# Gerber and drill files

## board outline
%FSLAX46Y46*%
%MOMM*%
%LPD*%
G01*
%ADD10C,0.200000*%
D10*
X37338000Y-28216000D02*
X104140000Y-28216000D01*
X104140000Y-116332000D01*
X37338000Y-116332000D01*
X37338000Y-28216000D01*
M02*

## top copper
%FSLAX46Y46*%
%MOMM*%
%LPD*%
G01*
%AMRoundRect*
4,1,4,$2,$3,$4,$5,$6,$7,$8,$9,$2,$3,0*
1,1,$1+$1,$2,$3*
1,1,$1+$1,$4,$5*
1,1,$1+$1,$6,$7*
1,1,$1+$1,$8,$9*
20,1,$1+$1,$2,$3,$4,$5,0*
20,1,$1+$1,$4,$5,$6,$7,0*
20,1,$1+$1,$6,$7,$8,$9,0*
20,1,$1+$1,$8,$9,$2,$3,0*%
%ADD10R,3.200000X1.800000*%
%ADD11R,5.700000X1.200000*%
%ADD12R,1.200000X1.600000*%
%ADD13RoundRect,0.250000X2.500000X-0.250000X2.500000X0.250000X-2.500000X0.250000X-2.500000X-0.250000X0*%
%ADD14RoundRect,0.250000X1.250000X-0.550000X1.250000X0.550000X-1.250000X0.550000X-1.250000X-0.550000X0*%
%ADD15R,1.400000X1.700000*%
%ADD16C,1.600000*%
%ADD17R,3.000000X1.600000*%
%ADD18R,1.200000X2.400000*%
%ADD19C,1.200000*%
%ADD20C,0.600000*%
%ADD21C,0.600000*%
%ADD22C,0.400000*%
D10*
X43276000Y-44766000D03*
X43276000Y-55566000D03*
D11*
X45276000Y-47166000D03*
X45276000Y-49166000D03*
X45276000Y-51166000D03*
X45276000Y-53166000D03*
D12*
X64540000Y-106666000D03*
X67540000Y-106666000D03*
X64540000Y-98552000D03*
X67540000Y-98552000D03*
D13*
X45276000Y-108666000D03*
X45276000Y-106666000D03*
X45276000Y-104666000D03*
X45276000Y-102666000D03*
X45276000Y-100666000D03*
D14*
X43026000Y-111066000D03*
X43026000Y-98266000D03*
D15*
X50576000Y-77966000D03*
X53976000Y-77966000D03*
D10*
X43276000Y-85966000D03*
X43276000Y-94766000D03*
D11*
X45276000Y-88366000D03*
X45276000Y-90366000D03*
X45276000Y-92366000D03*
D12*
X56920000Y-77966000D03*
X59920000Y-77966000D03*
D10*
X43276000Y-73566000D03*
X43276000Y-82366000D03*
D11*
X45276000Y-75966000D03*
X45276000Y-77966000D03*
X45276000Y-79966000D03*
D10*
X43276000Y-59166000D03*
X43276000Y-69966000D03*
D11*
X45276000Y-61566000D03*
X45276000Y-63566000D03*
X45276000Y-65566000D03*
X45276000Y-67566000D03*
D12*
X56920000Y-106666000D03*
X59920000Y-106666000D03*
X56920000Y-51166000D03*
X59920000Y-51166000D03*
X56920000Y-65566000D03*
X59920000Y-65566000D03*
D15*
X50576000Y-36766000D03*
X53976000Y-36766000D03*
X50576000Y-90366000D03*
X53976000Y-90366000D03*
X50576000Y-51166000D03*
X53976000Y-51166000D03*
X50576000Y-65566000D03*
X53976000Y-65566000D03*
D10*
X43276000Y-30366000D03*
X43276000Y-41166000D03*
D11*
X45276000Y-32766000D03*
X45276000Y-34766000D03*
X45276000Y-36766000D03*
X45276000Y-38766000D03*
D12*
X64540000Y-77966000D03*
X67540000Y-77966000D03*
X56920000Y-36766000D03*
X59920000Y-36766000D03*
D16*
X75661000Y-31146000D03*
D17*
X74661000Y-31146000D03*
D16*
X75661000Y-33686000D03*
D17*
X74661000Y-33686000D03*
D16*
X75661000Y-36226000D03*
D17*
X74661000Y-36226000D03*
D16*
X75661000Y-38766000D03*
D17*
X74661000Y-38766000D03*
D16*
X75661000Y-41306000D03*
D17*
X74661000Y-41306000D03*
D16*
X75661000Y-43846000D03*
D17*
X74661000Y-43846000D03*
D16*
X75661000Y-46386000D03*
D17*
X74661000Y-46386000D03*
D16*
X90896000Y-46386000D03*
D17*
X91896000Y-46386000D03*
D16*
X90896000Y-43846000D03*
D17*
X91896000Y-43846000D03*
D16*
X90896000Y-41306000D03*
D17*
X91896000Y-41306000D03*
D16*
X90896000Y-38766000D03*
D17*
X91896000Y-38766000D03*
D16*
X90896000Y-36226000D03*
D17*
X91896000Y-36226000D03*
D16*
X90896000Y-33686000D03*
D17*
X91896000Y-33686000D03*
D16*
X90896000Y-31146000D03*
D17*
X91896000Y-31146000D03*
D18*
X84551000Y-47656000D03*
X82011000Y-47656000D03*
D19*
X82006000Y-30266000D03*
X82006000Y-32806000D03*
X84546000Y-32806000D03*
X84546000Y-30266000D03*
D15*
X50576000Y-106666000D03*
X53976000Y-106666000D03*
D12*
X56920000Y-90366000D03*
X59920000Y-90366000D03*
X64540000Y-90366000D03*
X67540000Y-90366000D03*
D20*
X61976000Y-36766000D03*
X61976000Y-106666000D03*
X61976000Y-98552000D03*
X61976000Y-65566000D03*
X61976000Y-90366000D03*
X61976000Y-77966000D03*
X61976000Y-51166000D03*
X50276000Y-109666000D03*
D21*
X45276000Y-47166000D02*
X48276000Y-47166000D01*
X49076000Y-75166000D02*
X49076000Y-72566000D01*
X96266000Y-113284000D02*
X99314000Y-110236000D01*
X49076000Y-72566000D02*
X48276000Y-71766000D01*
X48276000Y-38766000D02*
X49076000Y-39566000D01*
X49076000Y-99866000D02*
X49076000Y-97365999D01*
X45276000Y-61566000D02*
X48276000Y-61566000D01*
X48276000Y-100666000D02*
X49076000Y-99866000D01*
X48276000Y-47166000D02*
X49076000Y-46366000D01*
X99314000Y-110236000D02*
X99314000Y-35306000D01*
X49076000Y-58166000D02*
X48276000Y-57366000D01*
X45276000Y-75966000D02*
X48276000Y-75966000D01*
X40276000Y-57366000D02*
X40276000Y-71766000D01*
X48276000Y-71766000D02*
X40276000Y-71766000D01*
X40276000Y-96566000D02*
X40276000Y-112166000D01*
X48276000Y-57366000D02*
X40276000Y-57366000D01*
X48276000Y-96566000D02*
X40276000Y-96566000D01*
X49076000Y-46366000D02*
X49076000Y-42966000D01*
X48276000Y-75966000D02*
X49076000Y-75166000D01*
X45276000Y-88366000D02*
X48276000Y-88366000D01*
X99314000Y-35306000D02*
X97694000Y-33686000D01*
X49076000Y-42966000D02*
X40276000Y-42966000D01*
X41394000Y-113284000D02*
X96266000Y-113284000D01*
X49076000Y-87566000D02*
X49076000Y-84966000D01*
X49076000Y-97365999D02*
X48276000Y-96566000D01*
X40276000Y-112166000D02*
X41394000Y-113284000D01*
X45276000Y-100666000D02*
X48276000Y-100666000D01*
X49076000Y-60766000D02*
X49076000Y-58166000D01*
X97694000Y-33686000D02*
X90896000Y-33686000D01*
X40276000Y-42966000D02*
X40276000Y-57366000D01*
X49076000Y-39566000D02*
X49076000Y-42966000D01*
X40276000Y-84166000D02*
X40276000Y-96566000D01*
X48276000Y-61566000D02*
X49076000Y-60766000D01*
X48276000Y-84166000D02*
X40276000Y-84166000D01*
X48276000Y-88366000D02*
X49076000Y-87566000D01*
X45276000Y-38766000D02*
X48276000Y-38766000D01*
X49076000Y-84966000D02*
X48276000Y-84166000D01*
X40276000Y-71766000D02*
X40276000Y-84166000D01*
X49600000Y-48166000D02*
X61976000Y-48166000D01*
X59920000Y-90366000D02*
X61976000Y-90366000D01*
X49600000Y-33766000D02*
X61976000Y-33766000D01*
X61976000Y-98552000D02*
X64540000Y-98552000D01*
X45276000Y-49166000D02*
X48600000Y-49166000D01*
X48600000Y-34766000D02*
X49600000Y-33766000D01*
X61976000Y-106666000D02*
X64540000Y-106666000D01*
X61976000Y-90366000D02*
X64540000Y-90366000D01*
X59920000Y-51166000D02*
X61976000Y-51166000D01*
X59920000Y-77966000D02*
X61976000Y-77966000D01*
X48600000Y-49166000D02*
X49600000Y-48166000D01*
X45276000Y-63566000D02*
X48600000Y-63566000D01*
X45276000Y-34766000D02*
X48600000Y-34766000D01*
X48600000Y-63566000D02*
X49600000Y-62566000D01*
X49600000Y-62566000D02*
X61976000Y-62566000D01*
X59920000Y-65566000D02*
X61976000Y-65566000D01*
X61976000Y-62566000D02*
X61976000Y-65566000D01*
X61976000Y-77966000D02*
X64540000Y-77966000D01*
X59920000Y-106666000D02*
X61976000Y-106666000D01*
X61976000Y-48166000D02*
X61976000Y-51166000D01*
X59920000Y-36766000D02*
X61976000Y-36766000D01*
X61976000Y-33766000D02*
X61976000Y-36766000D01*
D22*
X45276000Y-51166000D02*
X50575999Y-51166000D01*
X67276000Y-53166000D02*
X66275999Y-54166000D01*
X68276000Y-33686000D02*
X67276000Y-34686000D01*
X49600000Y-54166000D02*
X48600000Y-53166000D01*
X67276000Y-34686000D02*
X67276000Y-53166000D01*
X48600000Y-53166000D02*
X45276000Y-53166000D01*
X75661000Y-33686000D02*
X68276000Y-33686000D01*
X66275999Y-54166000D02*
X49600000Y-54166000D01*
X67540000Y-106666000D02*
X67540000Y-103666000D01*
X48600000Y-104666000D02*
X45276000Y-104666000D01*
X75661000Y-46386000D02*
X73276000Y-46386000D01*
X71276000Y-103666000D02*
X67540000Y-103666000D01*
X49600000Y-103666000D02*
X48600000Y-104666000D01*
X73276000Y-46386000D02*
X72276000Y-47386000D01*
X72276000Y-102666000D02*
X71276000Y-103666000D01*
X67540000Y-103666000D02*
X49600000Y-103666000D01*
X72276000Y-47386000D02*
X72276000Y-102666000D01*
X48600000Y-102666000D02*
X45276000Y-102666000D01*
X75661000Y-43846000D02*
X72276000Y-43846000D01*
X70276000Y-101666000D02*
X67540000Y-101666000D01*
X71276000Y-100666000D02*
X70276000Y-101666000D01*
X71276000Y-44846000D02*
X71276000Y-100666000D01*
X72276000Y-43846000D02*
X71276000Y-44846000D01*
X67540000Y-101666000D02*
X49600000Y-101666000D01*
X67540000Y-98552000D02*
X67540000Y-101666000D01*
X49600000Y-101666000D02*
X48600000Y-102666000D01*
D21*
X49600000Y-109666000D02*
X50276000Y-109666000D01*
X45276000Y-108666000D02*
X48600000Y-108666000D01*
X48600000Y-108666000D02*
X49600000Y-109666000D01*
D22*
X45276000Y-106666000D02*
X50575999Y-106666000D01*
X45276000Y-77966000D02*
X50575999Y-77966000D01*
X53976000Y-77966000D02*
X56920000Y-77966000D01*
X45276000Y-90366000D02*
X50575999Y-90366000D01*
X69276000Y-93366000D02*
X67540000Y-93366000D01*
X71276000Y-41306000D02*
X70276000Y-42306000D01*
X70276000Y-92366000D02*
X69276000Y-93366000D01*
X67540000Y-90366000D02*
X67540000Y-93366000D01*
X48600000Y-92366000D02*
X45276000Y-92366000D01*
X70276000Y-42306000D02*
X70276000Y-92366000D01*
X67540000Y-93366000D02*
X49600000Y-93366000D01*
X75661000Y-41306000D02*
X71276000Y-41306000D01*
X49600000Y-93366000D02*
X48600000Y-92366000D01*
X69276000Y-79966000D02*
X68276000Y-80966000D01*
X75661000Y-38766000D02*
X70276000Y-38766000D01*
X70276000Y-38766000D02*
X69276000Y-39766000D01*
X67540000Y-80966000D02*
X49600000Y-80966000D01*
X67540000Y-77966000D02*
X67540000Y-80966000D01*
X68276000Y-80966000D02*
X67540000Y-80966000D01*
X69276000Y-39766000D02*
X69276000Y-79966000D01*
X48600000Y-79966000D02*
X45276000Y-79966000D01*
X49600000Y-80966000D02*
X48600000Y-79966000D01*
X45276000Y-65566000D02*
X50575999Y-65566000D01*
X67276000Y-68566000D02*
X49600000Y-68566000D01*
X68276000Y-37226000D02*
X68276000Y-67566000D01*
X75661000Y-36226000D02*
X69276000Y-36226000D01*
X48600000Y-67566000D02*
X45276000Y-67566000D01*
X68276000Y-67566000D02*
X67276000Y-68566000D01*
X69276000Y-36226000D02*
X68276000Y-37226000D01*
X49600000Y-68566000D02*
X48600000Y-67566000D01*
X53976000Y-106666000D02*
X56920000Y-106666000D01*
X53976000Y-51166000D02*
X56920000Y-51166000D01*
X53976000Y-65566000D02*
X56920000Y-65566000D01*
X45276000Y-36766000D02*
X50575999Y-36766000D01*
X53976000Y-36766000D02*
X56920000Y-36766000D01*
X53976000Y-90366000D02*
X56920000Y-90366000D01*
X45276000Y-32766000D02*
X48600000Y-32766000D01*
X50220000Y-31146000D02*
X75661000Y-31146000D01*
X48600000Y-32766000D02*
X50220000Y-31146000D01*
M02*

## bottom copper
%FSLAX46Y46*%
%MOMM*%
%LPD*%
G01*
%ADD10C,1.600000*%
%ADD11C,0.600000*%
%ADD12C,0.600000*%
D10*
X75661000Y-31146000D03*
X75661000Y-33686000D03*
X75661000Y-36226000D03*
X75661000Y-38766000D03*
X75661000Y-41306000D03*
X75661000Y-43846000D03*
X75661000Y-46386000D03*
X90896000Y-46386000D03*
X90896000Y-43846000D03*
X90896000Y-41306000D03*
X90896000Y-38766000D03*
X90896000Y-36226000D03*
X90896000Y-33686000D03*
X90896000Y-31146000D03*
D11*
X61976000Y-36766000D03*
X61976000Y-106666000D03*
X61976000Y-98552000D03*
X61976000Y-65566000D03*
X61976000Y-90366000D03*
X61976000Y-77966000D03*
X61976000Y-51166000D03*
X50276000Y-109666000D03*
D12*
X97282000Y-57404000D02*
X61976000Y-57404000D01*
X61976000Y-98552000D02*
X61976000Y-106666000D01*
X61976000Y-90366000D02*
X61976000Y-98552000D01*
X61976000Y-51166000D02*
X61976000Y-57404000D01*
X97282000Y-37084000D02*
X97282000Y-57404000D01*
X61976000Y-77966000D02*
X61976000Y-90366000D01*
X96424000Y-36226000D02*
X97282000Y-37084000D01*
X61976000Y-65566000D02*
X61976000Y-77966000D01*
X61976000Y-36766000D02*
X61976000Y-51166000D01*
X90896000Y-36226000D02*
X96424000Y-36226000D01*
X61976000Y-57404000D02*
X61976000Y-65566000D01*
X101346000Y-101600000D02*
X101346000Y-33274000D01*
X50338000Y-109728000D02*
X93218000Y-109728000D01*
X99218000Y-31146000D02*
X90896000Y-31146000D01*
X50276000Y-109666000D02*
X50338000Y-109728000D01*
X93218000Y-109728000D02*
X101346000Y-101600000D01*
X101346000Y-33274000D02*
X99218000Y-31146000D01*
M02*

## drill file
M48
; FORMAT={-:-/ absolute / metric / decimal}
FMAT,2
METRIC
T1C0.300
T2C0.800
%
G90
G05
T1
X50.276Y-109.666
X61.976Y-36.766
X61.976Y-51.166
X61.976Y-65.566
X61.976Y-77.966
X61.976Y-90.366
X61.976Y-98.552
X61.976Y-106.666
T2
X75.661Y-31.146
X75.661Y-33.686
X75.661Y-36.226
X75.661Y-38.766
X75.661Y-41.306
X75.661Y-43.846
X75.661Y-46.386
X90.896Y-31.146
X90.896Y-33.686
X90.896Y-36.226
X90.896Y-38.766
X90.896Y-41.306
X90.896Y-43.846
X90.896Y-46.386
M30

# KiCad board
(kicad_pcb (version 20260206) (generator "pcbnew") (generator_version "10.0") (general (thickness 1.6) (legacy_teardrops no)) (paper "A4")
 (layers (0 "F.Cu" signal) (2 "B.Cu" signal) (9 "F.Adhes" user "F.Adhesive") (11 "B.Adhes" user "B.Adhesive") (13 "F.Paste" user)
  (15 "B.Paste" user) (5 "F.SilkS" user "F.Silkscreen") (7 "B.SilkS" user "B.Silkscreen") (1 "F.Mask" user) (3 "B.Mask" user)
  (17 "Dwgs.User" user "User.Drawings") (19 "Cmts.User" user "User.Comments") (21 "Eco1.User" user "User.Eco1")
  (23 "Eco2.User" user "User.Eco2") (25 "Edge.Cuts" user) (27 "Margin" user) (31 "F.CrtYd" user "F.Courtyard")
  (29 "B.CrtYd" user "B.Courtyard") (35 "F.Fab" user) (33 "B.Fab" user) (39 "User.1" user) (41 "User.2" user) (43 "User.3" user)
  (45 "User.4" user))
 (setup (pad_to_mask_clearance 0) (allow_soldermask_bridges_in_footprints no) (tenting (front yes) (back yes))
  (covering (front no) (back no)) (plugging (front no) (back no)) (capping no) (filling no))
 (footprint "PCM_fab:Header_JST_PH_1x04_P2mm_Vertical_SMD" (layer "F.Cu") (at 45.276 48.166)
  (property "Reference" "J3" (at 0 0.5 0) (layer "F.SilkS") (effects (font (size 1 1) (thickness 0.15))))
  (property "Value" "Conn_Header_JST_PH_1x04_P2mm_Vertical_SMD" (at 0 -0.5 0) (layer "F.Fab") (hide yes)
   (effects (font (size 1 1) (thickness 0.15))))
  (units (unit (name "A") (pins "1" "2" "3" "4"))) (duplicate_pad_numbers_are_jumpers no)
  (pad "" smd rect (at -2 -3.4) (size 3.2 1.8) (layers "F.Cu" "F.Mask" "F.Paste"))
  (pad "" smd rect (at -2 7.4) (size 3.2 1.8) (layers "F.Cu" "F.Mask" "F.Paste"))
  (pad "1" smd rect (at 0 -1) (size 5.7 1.2) (layers "F.Cu" "F.Mask" "F.Paste") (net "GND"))
  (pad "2" smd rect (at 0 1) (size 5.7 1.2) (layers "F.Cu" "F.Mask" "F.Paste") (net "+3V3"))
  (pad "3" smd rect (at 0 3) (size 5.7 1.2) (layers "F.Cu" "F.Mask" "F.Paste") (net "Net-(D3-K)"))
  (pad "4" smd rect (at 0 5) (size 5.7 1.2) (layers "F.Cu" "F.Mask" "F.Paste") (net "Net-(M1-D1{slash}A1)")))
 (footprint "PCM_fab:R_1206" (layer "F.Cu") (at 66.04 106.666)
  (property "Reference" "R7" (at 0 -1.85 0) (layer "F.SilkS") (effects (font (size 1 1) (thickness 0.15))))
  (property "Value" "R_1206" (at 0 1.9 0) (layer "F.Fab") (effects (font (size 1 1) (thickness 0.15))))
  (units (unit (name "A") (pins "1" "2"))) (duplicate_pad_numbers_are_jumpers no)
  (pad "1" smd rect (at -1.5 0) (size 1.2 1.6) (layers "F.Cu" "F.Mask" "F.Paste") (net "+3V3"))
  (pad "2" smd rect (at 1.5 0) (size 1.2 1.6) (layers "F.Cu" "F.Mask" "F.Paste") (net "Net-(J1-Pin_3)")))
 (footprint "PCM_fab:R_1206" (layer "F.Cu") (at 66.04 98.552)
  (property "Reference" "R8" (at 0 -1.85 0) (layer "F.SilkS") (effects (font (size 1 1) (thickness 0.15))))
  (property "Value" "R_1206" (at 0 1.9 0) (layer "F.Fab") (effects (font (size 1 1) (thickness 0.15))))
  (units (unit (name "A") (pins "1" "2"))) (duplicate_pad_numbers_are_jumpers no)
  (pad "1" smd rect (at -1.5 0) (size 1.2 1.6) (layers "F.Cu" "F.Mask" "F.Paste") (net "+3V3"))
  (pad "2" smd rect (at 1.5 0) (size 1.2 1.6) (layers "F.Cu" "F.Mask" "F.Paste") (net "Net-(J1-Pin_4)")))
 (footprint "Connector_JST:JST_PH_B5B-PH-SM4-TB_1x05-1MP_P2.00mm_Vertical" (layer "F.Cu") (at 44.776 104.666 90)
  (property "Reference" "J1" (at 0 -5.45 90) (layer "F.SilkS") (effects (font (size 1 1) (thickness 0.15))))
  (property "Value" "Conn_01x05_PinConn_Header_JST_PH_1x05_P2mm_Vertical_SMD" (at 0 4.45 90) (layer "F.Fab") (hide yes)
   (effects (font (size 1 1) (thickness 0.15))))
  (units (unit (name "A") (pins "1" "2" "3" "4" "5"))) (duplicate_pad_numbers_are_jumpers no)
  (pad "1" smd roundrect (at -4 0.5 90) (size 1 5.5) (layers "F.Cu" "F.Mask" "F.Paste") (roundrect_rratio 0.25) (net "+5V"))
  (pad "2" smd roundrect (at -2 0.5 90) (size 1 5.5) (layers "F.Cu" "F.Mask" "F.Paste") (roundrect_rratio 0.25) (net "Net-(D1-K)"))
  (pad "3" smd roundrect (at 0 0.5 90) (size 1 5.5) (layers "F.Cu" "F.Mask" "F.Paste") (roundrect_rratio 0.25) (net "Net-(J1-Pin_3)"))
  (pad "4" smd roundrect (at 2 0.5 90) (size 1 5.5) (layers "F.Cu" "F.Mask" "F.Paste") (roundrect_rratio 0.25) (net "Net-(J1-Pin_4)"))
  (pad "5" smd roundrect (at 4 0.5 90) (size 1 5.5) (layers "F.Cu" "F.Mask" "F.Paste") (roundrect_rratio 0.25) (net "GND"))
  (pad "MP" smd roundrect (at -6.4 -1.75 90) (size 1.6 3) (layers "F.Cu" "F.Mask" "F.Paste") (roundrect_rratio 0.15625))
  (pad "MP" smd roundrect (at 6.4 -1.75 90) (size 1.6 3) (layers "F.Cu" "F.Mask" "F.Paste") (roundrect_rratio 0.15625)))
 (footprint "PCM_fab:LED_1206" (layer "F.Cu") (at 52.276 77.966)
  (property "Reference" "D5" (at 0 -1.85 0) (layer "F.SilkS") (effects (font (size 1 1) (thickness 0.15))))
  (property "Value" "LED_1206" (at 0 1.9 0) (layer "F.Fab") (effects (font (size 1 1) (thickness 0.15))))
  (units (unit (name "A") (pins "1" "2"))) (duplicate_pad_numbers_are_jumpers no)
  (pad "1" smd rect (at -1.7 0) (size 1.4 1.7) (layers "F.Cu" "F.Mask" "F.Paste") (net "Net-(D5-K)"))
  (pad "2" smd rect (at 1.7 0) (size 1.4 1.7) (layers "F.Cu" "F.Mask" "F.Paste") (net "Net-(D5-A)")))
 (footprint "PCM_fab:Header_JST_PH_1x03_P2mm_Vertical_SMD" (layer "F.Cu") (at 45.276 89.366)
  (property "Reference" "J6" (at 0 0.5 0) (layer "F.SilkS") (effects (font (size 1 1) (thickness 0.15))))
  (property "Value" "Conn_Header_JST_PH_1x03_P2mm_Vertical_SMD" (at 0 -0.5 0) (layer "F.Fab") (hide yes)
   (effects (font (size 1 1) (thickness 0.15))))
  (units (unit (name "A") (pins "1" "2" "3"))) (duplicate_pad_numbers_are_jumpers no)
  (pad "" smd rect (at -2 -3.4) (size 3.2 1.8) (layers "F.Cu" "F.Mask" "F.Paste"))
  (pad "" smd rect (at -2 5.4) (size 3.2 1.8) (layers "F.Cu" "F.Mask" "F.Paste"))
  (pad "1" smd rect (at 0 -1) (size 5.7 1.2) (layers "F.Cu" "F.Mask" "F.Paste") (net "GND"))
  (pad "2" smd rect (at 0 1) (size 5.7 1.2) (layers "F.Cu" "F.Mask" "F.Paste") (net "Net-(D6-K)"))
  (pad "3" smd rect (at 0 3) (size 5.7 1.2) (layers "F.Cu" "F.Mask" "F.Paste") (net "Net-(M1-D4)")))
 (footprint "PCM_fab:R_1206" (layer "F.Cu") (at 58.42 77.966)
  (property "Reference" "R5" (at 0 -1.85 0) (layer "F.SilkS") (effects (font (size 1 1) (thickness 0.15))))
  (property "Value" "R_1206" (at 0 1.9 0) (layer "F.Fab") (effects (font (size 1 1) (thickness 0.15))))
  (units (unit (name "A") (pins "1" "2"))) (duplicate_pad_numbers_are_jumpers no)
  (pad "1" smd rect (at -1.5 0) (size 1.2 1.6) (layers "F.Cu" "F.Mask" "F.Paste") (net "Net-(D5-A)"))
  (pad "2" smd rect (at 1.5 0) (size 1.2 1.6) (layers "F.Cu" "F.Mask" "F.Paste") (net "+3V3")))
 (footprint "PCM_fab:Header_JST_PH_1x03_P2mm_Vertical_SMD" (layer "F.Cu") (at 45.276 76.966)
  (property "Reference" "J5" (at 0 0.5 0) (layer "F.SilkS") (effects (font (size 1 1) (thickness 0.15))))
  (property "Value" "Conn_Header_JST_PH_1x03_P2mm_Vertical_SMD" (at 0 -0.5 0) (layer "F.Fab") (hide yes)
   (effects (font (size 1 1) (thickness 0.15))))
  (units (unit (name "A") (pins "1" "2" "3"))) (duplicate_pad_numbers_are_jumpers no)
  (pad "" smd rect (at -2 -3.4) (size 3.2 1.8) (layers "F.Cu" "F.Mask" "F.Paste"))
  (pad "" smd rect (at -2 5.4) (size 3.2 1.8) (layers "F.Cu" "F.Mask" "F.Paste"))
  (pad "1" smd rect (at 0 -1) (size 5.7 1.2) (layers "F.Cu" "F.Mask" "F.Paste") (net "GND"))
  (pad "2" smd rect (at 0 1) (size 5.7 1.2) (layers "F.Cu" "F.Mask" "F.Paste") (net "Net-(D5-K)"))
  (pad "3" smd rect (at 0 3) (size 5.7 1.2) (layers "F.Cu" "F.Mask" "F.Paste") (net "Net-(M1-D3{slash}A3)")))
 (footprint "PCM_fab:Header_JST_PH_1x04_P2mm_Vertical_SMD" (layer "F.Cu") (at 45.276 62.566)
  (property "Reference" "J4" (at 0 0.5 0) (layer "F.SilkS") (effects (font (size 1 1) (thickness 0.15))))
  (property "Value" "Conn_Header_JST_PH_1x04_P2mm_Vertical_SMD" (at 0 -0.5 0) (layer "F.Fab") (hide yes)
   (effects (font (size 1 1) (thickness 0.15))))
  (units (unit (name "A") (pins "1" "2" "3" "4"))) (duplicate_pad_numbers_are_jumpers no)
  (pad "" smd rect (at -2 -3.4) (size 3.2 1.8) (layers "F.Cu" "F.Mask" "F.Paste"))
  (pad "" smd rect (at -2 7.4) (size 3.2 1.8) (layers "F.Cu" "F.Mask" "F.Paste"))
  (pad "1" smd rect (at 0 -1) (size 5.7 1.2) (layers "F.Cu" "F.Mask" "F.Paste") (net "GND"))
  (pad "2" smd rect (at 0 1) (size 5.7 1.2) (layers "F.Cu" "F.Mask" "F.Paste") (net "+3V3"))
  (pad "3" smd rect (at 0 3) (size 5.7 1.2) (layers "F.Cu" "F.Mask" "F.Paste") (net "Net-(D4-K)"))
  (pad "4" smd rect (at 0 5) (size 5.7 1.2) (layers "F.Cu" "F.Mask" "F.Paste") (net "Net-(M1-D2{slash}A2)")))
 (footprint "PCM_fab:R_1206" (layer "F.Cu") (at 58.42 106.666)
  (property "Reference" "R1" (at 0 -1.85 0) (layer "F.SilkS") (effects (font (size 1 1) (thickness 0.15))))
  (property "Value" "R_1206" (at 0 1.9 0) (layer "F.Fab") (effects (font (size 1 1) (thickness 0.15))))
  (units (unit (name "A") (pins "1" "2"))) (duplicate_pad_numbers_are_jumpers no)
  (pad "1" smd rect (at -1.5 0) (size 1.2 1.6) (layers "F.Cu" "F.Mask" "F.Paste") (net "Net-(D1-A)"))
  (pad "2" smd rect (at 1.5 0) (size 1.2 1.6) (layers "F.Cu" "F.Mask" "F.Paste") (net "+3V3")))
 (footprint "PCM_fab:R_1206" (layer "F.Cu") (at 58.42 51.166)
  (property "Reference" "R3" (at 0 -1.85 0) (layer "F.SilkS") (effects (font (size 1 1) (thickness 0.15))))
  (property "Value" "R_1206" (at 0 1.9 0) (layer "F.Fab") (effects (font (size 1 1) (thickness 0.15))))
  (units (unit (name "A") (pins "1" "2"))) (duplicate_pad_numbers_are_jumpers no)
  (pad "1" smd rect (at -1.5 0) (size 1.2 1.6) (layers "F.Cu" "F.Mask" "F.Paste") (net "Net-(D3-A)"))
  (pad "2" smd rect (at 1.5 0) (size 1.2 1.6) (layers "F.Cu" "F.Mask" "F.Paste") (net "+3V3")))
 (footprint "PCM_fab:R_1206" (layer "F.Cu") (at 58.42 65.566)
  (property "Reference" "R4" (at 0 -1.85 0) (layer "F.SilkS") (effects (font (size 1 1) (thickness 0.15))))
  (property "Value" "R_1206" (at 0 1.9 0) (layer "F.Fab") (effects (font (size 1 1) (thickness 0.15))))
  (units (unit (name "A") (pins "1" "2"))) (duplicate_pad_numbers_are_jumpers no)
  (pad "1" smd rect (at -1.5 0) (size 1.2 1.6) (layers "F.Cu" "F.Mask" "F.Paste") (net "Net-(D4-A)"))
  (pad "2" smd rect (at 1.5 0) (size 1.2 1.6) (layers "F.Cu" "F.Mask" "F.Paste") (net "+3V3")))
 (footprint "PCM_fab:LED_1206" (layer "F.Cu") (at 52.276 36.766)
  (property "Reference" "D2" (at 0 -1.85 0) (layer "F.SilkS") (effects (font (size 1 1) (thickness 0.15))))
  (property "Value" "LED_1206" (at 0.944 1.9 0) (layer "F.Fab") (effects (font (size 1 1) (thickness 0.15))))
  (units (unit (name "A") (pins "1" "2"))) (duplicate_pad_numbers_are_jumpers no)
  (pad "1" smd rect (at -1.7 0) (size 1.4 1.7) (layers "F.Cu" "F.Mask" "F.Paste") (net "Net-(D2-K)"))
  (pad "2" smd rect (at 1.7 0) (size 1.4 1.7) (layers "F.Cu" "F.Mask" "F.Paste") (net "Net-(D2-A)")))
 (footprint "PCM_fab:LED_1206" (layer "F.Cu") (at 52.276 90.366)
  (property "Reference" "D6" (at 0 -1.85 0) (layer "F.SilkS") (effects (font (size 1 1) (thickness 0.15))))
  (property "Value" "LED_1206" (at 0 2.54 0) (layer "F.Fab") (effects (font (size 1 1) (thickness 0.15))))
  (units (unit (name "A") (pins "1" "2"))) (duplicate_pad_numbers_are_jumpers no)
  (pad "1" smd rect (at -1.7 0) (size 1.4 1.7) (layers "F.Cu" "F.Mask" "F.Paste") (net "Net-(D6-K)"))
  (pad "2" smd rect (at 1.7 0) (size 1.4 1.7) (layers "F.Cu" "F.Mask" "F.Paste") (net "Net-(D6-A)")))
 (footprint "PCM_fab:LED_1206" (layer "F.Cu") (at 52.276 51.166)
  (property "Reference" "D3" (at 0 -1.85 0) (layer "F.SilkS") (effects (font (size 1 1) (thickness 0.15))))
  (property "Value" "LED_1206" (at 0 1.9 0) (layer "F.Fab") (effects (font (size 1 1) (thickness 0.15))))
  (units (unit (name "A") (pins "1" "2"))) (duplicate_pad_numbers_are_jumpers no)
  (pad "1" smd rect (at -1.7 0) (size 1.4 1.7) (layers "F.Cu" "F.Mask" "F.Paste") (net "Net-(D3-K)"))
  (pad "2" smd rect (at 1.7 0) (size 1.4 1.7) (layers "F.Cu" "F.Mask" "F.Paste") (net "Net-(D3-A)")))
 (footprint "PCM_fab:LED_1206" (layer "F.Cu") (at 52.276 65.566)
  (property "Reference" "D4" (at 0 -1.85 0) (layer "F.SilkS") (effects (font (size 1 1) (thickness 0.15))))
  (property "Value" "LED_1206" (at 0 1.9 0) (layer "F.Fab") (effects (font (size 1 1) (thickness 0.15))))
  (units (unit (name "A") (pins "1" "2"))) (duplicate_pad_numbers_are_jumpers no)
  (pad "1" smd rect (at -1.7 0) (size 1.4 1.7) (layers "F.Cu" "F.Mask" "F.Paste") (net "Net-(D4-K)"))
  (pad "2" smd rect (at 1.7 0) (size 1.4 1.7) (layers "F.Cu" "F.Mask" "F.Paste") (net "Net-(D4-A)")))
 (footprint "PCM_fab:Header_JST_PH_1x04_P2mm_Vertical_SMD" (layer "F.Cu") (at 45.276 33.766)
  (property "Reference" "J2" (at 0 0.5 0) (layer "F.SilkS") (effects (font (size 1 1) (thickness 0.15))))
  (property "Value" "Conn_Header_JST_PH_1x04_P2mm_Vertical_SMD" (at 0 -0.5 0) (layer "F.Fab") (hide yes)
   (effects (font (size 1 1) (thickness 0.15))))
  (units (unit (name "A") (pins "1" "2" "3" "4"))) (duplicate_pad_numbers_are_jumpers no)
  (pad "" smd rect (at -2 -3.4) (size 3.2 1.8) (layers "F.Cu" "F.Mask" "F.Paste"))
  (pad "" smd rect (at -2 7.4) (size 3.2 1.8) (layers "F.Cu" "F.Mask" "F.Paste"))
  (pad "1" smd rect (at 0 -1) (size 5.7 1.2) (layers "F.Cu" "F.Mask" "F.Paste") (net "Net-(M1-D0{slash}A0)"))
  (pad "2" smd rect (at 0 1) (size 5.7 1.2) (layers "F.Cu" "F.Mask" "F.Paste") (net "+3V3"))
  (pad "3" smd rect (at 0 3) (size 5.7 1.2) (layers "F.Cu" "F.Mask" "F.Paste") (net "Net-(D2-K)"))
  (pad "4" smd rect (at 0 5) (size 5.7 1.2) (layers "F.Cu" "F.Mask" "F.Paste") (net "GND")))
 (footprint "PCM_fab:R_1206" (layer "F.Cu") (at 66.04 77.966)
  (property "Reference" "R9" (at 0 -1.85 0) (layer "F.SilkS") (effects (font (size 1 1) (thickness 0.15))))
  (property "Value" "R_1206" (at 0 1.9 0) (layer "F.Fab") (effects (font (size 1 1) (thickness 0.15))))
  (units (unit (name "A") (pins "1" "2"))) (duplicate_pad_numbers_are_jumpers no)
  (pad "1" smd rect (at -1.5 0) (size 1.2 1.6) (layers "F.Cu" "F.Mask" "F.Paste") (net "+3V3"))
  (pad "2" smd rect (at 1.5 0) (size 1.2 1.6) (layers "F.Cu" "F.Mask" "F.Paste") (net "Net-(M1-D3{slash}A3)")))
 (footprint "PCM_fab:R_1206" (layer "F.Cu") (at 58.42 36.766)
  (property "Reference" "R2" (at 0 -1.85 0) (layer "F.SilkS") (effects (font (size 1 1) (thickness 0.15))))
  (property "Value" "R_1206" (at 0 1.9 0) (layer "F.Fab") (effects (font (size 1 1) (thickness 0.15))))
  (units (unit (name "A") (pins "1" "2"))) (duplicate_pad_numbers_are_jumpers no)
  (pad "1" smd rect (at -1.5 0) (size 1.2 1.6) (layers "F.Cu" "F.Mask" "F.Paste") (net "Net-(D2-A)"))
  (pad "2" smd rect (at 1.5 0) (size 1.2 1.6) (layers "F.Cu" "F.Mask" "F.Paste") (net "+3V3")))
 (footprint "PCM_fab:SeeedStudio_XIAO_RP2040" (layer "F.Cu") (at 83.276 38.766)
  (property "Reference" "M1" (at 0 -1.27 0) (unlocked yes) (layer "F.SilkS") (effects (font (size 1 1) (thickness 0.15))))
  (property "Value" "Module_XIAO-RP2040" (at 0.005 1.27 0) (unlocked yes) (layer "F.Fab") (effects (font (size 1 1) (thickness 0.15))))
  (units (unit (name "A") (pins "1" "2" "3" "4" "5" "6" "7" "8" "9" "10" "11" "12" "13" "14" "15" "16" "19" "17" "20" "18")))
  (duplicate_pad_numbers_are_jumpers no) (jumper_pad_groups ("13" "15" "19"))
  (pad "1" thru_hole circle (at -7.615 -7.62) (size 1.6 1.6) (drill 0.8) (layers "*.Cu" "*.Mask") (remove_unused_layers no)
   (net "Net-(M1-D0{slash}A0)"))
  (pad "1" smd rect (at -7.615 -7.62) (size 3 1.6) (drill (offset -1 0)) (layers "F.Cu" "F.Mask" "F.Paste") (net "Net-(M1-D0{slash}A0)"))
  (pad "2" thru_hole circle (at -7.615 -5.08) (size 1.6 1.6) (drill 0.8) (layers "*.Cu" "*.Mask") (remove_unused_layers no)
   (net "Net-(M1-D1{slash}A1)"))
  (pad "2" smd rect (at -7.615 -5.08) (size 3 1.6) (drill (offset -1 0)) (layers "F.Cu" "F.Mask" "F.Paste") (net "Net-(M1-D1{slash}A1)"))
  (pad "3" thru_hole circle (at -7.615 -2.54) (size 1.6 1.6) (drill 0.8) (layers "*.Cu" "*.Mask") (remove_unused_layers no)
   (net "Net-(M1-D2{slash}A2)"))
  (pad "3" smd rect (at -7.615 -2.54) (size 3 1.6) (drill (offset -1 0)) (layers "F.Cu" "F.Mask" "F.Paste") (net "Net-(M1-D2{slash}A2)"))
  (pad "4" thru_hole circle (at -7.615 0) (size 1.6 1.6) (drill 0.8) (layers "*.Cu" "*.Mask") (remove_unused_layers no)
   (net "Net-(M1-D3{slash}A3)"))
  (pad "4" smd rect (at -7.615 0) (size 3 1.6) (drill (offset -1 0)) (layers "F.Cu" "F.Mask" "F.Paste") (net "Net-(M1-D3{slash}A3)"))
  (pad "5" thru_hole circle (at -7.615 2.54) (size 1.6 1.6) (drill 0.8) (layers "*.Cu" "*.Mask") (remove_unused_layers no)
   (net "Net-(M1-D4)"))
  (pad "5" smd rect (at -7.615 2.54) (size 3 1.6) (drill (offset -1 0)) (layers "F.Cu" "F.Mask" "F.Paste") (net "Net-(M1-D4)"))
  (pad "6" thru_hole circle (at -7.615 5.08) (size 1.6 1.6) (drill 0.8) (layers "*.Cu" "*.Mask") (remove_unused_layers no)
   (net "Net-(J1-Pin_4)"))
  (pad "6" smd rect (at -7.615 5.08) (size 3 1.6) (drill (offset -1 0)) (layers "F.Cu" "F.Mask" "F.Paste") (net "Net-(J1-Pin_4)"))
  (pad "7" thru_hole circle (at -7.615 7.62) (size 1.6 1.6) (drill 0.8) (layers "*.Cu" "*.Mask") (remove_unused_layers no)
   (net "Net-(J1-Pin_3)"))
  (pad "7" smd rect (at -7.615 7.62) (size 3 1.6) (drill (offset -1 0)) (layers "F.Cu" "F.Mask" "F.Paste") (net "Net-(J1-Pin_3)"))
  (pad "8" thru_hole circle (at 7.62 7.62) (size 1.6 1.6) (drill 0.8) (layers "*.Cu" "*.Mask") (remove_unused_layers no)
   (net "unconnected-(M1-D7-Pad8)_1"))
  (pad "8" smd rect (at 7.62 7.62) (size 3 1.6) (drill (offset 1 0)) (layers "F.Cu" "F.Mask" "F.Paste") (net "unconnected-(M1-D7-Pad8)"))
  (pad "9" thru_hole circle (at 7.62 5.08) (size 1.6 1.6) (drill 0.8) (layers "*.Cu" "*.Mask") (remove_unused_layers no)
   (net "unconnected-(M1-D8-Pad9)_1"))
  (pad "9" smd rect (at 7.62 5.08) (size 3 1.6) (drill (offset 1 0)) (layers "F.Cu" "F.Mask" "F.Paste") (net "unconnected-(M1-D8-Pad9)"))
  (pad "10" thru_hole circle (at 7.62 2.54) (size 1.6 1.6) (drill 0.8) (layers "*.Cu" "*.Mask") (remove_unused_layers no)
   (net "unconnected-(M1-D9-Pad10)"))
  (pad "10" smd rect (at 7.62 2.54) (size 3 1.6) (drill (offset 1 0)) (layers "F.Cu" "F.Mask" "F.Paste") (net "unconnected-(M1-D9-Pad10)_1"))
  (pad "11" thru_hole circle (at 7.62 0) (size 1.6 1.6) (drill 0.8) (layers "*.Cu" "*.Mask") (remove_unused_layers no)
   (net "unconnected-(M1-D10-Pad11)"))
  (pad "11" smd rect (at 7.62 0) (size 3 1.6) (drill (offset 1 0)) (layers "F.Cu" "F.Mask" "F.Paste") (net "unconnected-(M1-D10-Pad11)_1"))
  (pad "12" thru_hole circle (at 7.62 -2.54) (size 1.6 1.6) (drill 0.8) (layers "*.Cu" "*.Mask") (remove_unused_layers no) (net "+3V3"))
  (pad "12" smd rect (at 7.62 -2.54) (size 3 1.6) (drill (offset 1 0)) (layers "F.Cu" "F.Mask" "F.Paste") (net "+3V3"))
  (pad "13" thru_hole circle (at 7.62 -5.08) (size 1.6 1.6) (drill 0.8) (layers "*.Cu" "*.Mask") (remove_unused_layers no) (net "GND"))
  (pad "13" smd rect (at 7.62 -5.08) (size 3 1.6) (drill (offset 1 0)) (layers "F.Cu" "F.Mask" "F.Paste") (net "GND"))
  (pad "14" thru_hole circle (at 7.62 -7.62) (size 1.6 1.6) (drill 0.8) (layers "*.Cu" "*.Mask") (remove_unused_layers no) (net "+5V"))
  (pad "14" smd rect (at 7.62 -7.62) (size 3 1.6) (drill (offset 1 0)) (layers "F.Cu" "F.Mask" "F.Paste") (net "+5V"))
  (pad "15" smd rect (at 1.275 8.89 270) (size 2.4 1.2) (layers "F.Cu" "F.Mask" "F.Paste") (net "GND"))
  (pad "16" smd rect (at -1.265 8.89 270) (size 2.4 1.2) (layers "F.Cu" "F.Mask" "F.Paste") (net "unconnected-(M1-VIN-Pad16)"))
  (pad "17" smd circle (at -1.27 -8.5) (size 1.2 1.2) (layers "F.Cu" "F.Mask" "F.Paste") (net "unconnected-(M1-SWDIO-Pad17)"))
  (pad "18" smd circle (at -1.27 -5.96) (size 1.2 1.2) (layers "F.Cu" "F.Mask" "F.Paste") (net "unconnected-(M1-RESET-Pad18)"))
  (pad "19" smd circle (at 1.27 -5.96) (size 1.2 1.2) (layers "F.Cu" "F.Mask" "F.Paste") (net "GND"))
  (pad "20" smd circle (at 1.27 -8.5) (size 1.2 1.2) (layers "F.Cu" "F.Mask" "F.Paste") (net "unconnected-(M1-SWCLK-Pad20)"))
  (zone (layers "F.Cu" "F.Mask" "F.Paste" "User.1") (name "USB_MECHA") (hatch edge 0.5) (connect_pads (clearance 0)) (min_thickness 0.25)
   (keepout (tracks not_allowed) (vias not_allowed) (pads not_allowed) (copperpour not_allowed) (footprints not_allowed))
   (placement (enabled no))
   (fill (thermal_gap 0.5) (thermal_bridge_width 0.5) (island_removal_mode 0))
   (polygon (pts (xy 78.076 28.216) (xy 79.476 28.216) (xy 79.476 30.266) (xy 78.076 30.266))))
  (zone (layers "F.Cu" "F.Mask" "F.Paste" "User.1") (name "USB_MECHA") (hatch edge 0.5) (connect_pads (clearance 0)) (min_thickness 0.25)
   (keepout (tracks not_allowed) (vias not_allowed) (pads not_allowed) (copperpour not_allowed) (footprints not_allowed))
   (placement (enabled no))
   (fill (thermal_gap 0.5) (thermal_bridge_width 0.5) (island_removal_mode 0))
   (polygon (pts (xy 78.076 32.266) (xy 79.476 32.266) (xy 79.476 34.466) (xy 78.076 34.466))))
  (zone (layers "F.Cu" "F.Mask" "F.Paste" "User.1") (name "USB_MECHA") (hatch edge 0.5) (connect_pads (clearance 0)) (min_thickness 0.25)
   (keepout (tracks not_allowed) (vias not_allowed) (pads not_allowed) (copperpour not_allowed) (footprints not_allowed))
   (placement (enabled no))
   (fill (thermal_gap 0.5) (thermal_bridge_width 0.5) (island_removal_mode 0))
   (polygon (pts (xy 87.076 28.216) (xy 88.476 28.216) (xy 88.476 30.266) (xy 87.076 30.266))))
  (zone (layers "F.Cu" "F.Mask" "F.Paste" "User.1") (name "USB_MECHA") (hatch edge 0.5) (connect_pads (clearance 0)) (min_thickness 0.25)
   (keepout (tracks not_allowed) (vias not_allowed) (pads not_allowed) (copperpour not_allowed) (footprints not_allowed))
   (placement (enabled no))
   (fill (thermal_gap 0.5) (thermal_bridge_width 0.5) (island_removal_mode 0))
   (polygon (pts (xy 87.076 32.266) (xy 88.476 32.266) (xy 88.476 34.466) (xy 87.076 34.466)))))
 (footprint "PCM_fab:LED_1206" (layer "F.Cu") (at 52.276 106.666)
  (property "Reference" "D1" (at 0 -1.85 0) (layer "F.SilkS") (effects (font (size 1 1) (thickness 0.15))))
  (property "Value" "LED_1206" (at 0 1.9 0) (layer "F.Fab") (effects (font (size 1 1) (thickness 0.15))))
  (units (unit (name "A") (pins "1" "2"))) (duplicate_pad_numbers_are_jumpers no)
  (pad "1" smd rect (at -1.7 0) (size 1.4 1.7) (layers "F.Cu" "F.Mask" "F.Paste") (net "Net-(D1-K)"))
  (pad "2" smd rect (at 1.7 0) (size 1.4 1.7) (layers "F.Cu" "F.Mask" "F.Paste") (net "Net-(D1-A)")))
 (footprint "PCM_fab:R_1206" (layer "F.Cu") (at 58.42 90.366)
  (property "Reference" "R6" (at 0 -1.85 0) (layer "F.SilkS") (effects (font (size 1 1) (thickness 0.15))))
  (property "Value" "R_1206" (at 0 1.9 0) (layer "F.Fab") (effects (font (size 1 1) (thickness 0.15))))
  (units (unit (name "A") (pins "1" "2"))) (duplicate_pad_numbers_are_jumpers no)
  (pad "1" smd rect (at -1.5 0) (size 1.2 1.6) (layers "F.Cu" "F.Mask" "F.Paste") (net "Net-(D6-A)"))
  (pad "2" smd rect (at 1.5 0) (size 1.2 1.6) (layers "F.Cu" "F.Mask" "F.Paste") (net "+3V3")))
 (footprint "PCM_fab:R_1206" (layer "F.Cu") (at 66.04 90.366)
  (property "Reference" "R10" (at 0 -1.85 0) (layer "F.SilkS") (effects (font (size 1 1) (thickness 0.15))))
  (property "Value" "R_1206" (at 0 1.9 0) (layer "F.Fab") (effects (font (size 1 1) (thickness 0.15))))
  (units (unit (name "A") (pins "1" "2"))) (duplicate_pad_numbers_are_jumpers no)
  (pad "1" smd rect (at -1.5 0) (size 1.2 1.6) (layers "F.Cu" "F.Mask" "F.Paste") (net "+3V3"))
  (pad "2" smd rect (at 1.5 0) (size 1.2 1.6) (layers "F.Cu" "F.Mask" "F.Paste") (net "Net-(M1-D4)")))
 (gr_rect (start 37.338 28.216) (end 104.14 116.332) (stroke (width 0.2) (type solid)) (fill no) (layer "Edge.Cuts"))
 (segment (start 45.276 47.166) (end 48.276 47.166) (width 0.6) (layer "F.Cu") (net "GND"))
 (segment (start 49.076 75.166) (end 49.076 72.566) (width 0.6) (layer "F.Cu") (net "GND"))
 (segment (start 96.266 113.284) (end 99.314 110.236) (width 0.6) (layer "F.Cu") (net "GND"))
 (segment (start 49.076 72.566) (end 48.276 71.766) (width 0.6) (layer "F.Cu") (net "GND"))
 (segment (start 48.276 38.766) (end 49.076 39.566) (width 0.6) (layer "F.Cu") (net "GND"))
 (segment (start 49.076 99.866) (end 49.076 97.365999) (width 0.6) (layer "F.Cu") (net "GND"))
 (segment (start 45.276 61.566) (end 48.276 61.566) (width 0.6) (layer "F.Cu") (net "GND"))
 (segment (start 48.276 100.666) (end 49.076 99.866) (width 0.6) (layer "F.Cu") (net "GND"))
 (segment (start 48.276 47.166) (end 49.076 46.366) (width 0.6) (layer "F.Cu") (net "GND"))
 (segment (start 99.314 110.236) (end 99.314 35.306) (width 0.6) (layer "F.Cu") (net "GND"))
 (segment (start 49.076 58.166) (end 48.276 57.366) (width 0.6) (layer "F.Cu") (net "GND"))
 (segment (start 45.276 75.966) (end 48.276 75.966) (width 0.6) (layer "F.Cu") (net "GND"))
 (segment (start 40.276 57.366) (end 40.276 71.766) (width 0.6) (layer "F.Cu") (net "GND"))
 (segment (start 48.276 71.766) (end 40.276 71.766) (width 0.6) (layer "F.Cu") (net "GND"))
 (segment (start 40.276 96.566) (end 40.276 112.166) (width 0.6) (layer "F.Cu") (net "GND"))
 (segment (start 48.276 57.366) (end 40.276 57.366) (width 0.6) (layer "F.Cu") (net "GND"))
 (segment (start 48.276 96.566) (end 40.276 96.566) (width 0.6) (layer "F.Cu") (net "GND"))
 (segment (start 49.076 46.366) (end 49.076 42.966) (width 0.6) (layer "F.Cu") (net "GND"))
 (segment (start 48.276 75.966) (end 49.076 75.166) (width 0.6) (layer "F.Cu") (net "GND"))
 (segment (start 45.276 88.366) (end 48.276 88.366) (width 0.6) (layer "F.Cu") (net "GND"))
 (segment (start 99.314 35.306) (end 97.694 33.686) (width 0.6) (layer "F.Cu") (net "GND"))
 (segment (start 49.076 42.966) (end 40.276 42.966) (width 0.6) (layer "F.Cu") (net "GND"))
 (segment (start 41.394 113.284) (end 96.266 113.284) (width 0.6) (layer "F.Cu") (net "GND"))
 (segment (start 49.076 87.566) (end 49.076 84.966) (width 0.6) (layer "F.Cu") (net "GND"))
 (segment (start 49.076 97.365999) (end 48.276 96.566) (width 0.6) (layer "F.Cu") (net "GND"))
 (segment (start 40.276 112.166) (end 41.394 113.284) (width 0.6) (layer "F.Cu") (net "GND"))
 (segment (start 45.276 100.666) (end 48.276 100.666) (width 0.6) (layer "F.Cu") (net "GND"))
 (segment (start 49.076 60.766) (end 49.076 58.166) (width 0.6) (layer "F.Cu") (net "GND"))
 (segment (start 97.694 33.686) (end 90.896 33.686) (width 0.6) (layer "F.Cu") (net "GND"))
 (segment (start 40.276 42.966) (end 40.276 57.366) (width 0.6) (layer "F.Cu") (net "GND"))
 (segment (start 49.076 39.566) (end 49.076 42.966) (width 0.6) (layer "F.Cu") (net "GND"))
 (segment (start 40.276 84.166) (end 40.276 96.566) (width 0.6) (layer "F.Cu") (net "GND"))
 (segment (start 48.276 61.566) (end 49.076 60.766) (width 0.6) (layer "F.Cu") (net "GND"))
 (segment (start 48.276 84.166) (end 40.276 84.166) (width 0.6) (layer "F.Cu") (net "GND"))
 (segment (start 48.276 88.366) (end 49.076 87.566) (width 0.6) (layer "F.Cu") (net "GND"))
 (segment (start 45.276 38.766) (end 48.276 38.766) (width 0.6) (layer "F.Cu") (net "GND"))
 (segment (start 49.076 84.966) (end 48.276 84.166) (width 0.6) (layer "F.Cu") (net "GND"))
 (segment (start 40.276 71.766) (end 40.276 84.166) (width 0.6) (layer "F.Cu") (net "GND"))
 (segment (start 49.6 48.166) (end 61.976 48.166) (width 0.6) (layer "F.Cu") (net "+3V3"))
 (segment (start 59.92 90.366) (end 61.976 90.366) (width 0.6) (layer "F.Cu") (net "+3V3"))
 (segment (start 49.6 33.766) (end 61.976 33.766) (width 0.6) (layer "F.Cu") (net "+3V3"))
 (segment (start 61.976 98.552) (end 64.54 98.552) (width 0.6) (layer "F.Cu") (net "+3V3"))
 (segment (start 45.276 49.166) (end 48.6 49.166) (width 0.6) (layer "F.Cu") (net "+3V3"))
 (segment (start 48.6 34.766) (end 49.6 33.766) (width 0.6) (layer "F.Cu") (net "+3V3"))
 (segment (start 61.976 106.666) (end 64.54 106.666) (width 0.6) (layer "F.Cu") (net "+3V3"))
 (segment (start 61.976 90.366) (end 64.54 90.366) (width 0.6) (layer "F.Cu") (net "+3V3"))
 (segment (start 59.92 51.166) (end 61.976 51.166) (width 0.6) (layer "F.Cu") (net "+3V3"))
 (segment (start 59.92 77.966) (end 61.976 77.966) (width 0.6) (layer "F.Cu") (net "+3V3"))
 (segment (start 48.6 49.166) (end 49.6 48.166) (width 0.6) (layer "F.Cu") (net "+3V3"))
 (segment (start 45.276 63.566) (end 48.6 63.566) (width 0.6) (layer "F.Cu") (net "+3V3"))
 (segment (start 45.276 34.766) (end 48.6 34.766) (width 0.6) (layer "F.Cu") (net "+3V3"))
 (segment (start 48.6 63.566) (end 49.6 62.566) (width 0.6) (layer "F.Cu") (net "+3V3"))
 (segment (start 49.6 62.566) (end 61.976 62.566) (width 0.6) (layer "F.Cu") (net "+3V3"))
 (segment (start 59.92 65.566) (end 61.976 65.566) (width 0.6) (layer "F.Cu") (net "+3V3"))
 (segment (start 61.976 62.566) (end 61.976 65.566) (width 0.6) (layer "F.Cu") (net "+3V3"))
 (segment (start 61.976 77.966) (end 64.54 77.966) (width 0.6) (layer "F.Cu") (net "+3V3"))
 (segment (start 59.92 106.666) (end 61.976 106.666) (width 0.6) (layer "F.Cu") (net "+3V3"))
 (segment (start 61.976 48.166) (end 61.976 51.166) (width 0.6) (layer "F.Cu") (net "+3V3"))
 (segment (start 59.92 36.766) (end 61.976 36.766) (width 0.6) (layer "F.Cu") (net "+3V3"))
 (segment (start 61.976 33.766) (end 61.976 36.766) (width 0.6) (layer "F.Cu") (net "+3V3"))
 (via (at 61.976 36.766) (size 0.6) (drill 0.3) (layers "F.Cu" "B.Cu") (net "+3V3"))
 (via (at 61.976 106.666) (size 0.6) (drill 0.3) (layers "F.Cu" "B.Cu") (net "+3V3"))
 (via (at 61.976 98.552) (size 0.6) (drill 0.3) (layers "F.Cu" "B.Cu") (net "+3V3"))
 (via (at 61.976 65.566) (size 0.6) (drill 0.3) (layers "F.Cu" "B.Cu") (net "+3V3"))
 (via (at 61.976 90.366) (size 0.6) (drill 0.3) (layers "F.Cu" "B.Cu") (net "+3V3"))
 (via (at 61.976 77.966) (size 0.6) (drill 0.3) (layers "F.Cu" "B.Cu") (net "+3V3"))
 (via (at 61.976 51.166) (size 0.6) (drill 0.3) (layers "F.Cu" "B.Cu") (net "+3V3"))
 (segment (start 97.282 57.404) (end 61.976 57.404) (width 0.6) (layer "B.Cu") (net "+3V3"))
 (segment (start 61.976 98.552) (end 61.976 106.666) (width 0.6) (layer "B.Cu") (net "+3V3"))
 (segment (start 61.976 90.366) (end 61.976 98.552) (width 0.6) (layer "B.Cu") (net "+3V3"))
 (segment (start 61.976 51.166) (end 61.976 57.404) (width 0.6) (layer "B.Cu") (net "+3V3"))
 (segment (start 97.282 37.084) (end 97.282 57.404) (width 0.6) (layer "B.Cu") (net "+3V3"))
 (segment (start 61.976 77.966) (end 61.976 90.366) (width 0.6) (layer "B.Cu") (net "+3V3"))
 (segment (start 96.424 36.226) (end 97.282 37.084) (width 0.6) (layer "B.Cu") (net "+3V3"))
 (segment (start 61.976 65.566) (end 61.976 77.966) (width 0.6) (layer "B.Cu") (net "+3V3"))
 (segment (start 61.976 36.766) (end 61.976 51.166) (width 0.6) (layer "B.Cu") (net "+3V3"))
 (segment (start 90.896 36.226) (end 96.424 36.226) (width 0.6) (layer "B.Cu") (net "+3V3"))
 (segment (start 61.976 57.404) (end 61.976 65.566) (width 0.6) (layer "B.Cu") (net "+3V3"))
 (segment (start 45.276 51.166) (end 50.575999 51.166) (width 0.4) (layer "F.Cu") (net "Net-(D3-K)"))
 (segment (start 67.276 53.166) (end 66.275999 54.166) (width 0.4) (layer "F.Cu") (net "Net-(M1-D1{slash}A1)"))
 (segment (start 68.276 33.686) (end 67.276 34.686) (width 0.4) (layer "F.Cu") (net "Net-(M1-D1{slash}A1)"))
 (segment (start 49.6 54.166) (end 48.6 53.166) (width 0.4) (layer "F.Cu") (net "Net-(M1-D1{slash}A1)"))
 (segment (start 67.276 34.686) (end 67.276 53.166) (width 0.4) (layer "F.Cu") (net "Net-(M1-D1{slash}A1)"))
 (segment (start 48.6 53.166) (end 45.276 53.166) (width 0.4) (layer "F.Cu") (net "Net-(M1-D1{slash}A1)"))
 (segment (start 75.661 33.686) (end 68.276 33.686) (width 0.4) (layer "F.Cu") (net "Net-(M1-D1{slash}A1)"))
 (segment (start 66.275999 54.166) (end 49.6 54.166) (width 0.4) (layer "F.Cu") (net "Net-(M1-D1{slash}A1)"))
 (segment (start 67.54 106.666) (end 67.54 103.666) (width 0.4) (layer "F.Cu") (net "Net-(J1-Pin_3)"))
 (segment (start 48.6 104.666) (end 45.276 104.666) (width 0.4) (layer "F.Cu") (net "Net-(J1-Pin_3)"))
 (segment (start 75.661 46.386) (end 73.276 46.386) (width 0.4) (layer "F.Cu") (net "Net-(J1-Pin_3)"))
 (segment (start 71.276 103.666) (end 67.54 103.666) (width 0.4) (layer "F.Cu") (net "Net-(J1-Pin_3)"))
 (segment (start 49.6 103.666) (end 48.6 104.666) (width 0.4) (layer "F.Cu") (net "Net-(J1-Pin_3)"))
 (segment (start 73.276 46.386) (end 72.276 47.386) (width 0.4) (layer "F.Cu") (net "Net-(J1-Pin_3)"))
 (segment (start 72.276 102.666) (end 71.276 103.666) (width 0.4) (layer "F.Cu") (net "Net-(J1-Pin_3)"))
 (segment (start 67.54 103.666) (end 49.6 103.666) (width 0.4) (layer "F.Cu") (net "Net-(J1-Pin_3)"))
 (segment (start 72.276 47.386) (end 72.276 102.666) (width 0.4) (layer "F.Cu") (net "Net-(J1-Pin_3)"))
 (segment (start 48.6 102.666) (end 45.276 102.666) (width 0.4) (layer "F.Cu") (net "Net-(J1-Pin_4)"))
 (segment (start 75.661 43.846) (end 72.276 43.846) (width 0.4) (layer "F.Cu") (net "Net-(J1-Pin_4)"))
 (segment (start 70.276 101.666) (end 67.54 101.666) (width 0.4) (layer "F.Cu") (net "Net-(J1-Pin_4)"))
 (segment (start 71.276 100.666) (end 70.276 101.666) (width 0.4) (layer "F.Cu") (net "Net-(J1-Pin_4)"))
 (segment (start 71.276 44.846) (end 71.276 100.666) (width 0.4) (layer "F.Cu") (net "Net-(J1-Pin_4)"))
 (segment (start 72.276 43.846) (end 71.276 44.846) (width 0.4) (layer "F.Cu") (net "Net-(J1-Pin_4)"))
 (segment (start 67.54 101.666) (end 49.6 101.666) (width 0.4) (layer "F.Cu") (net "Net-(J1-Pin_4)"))
 (segment (start 67.54 98.552) (end 67.54 101.666) (width 0.4) (layer "F.Cu") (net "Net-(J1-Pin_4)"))
 (segment (start 49.6 101.666) (end 48.6 102.666) (width 0.4) (layer "F.Cu") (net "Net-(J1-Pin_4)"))
 (segment (start 49.6 109.666) (end 50.276 109.666) (width 0.6) (layer "F.Cu") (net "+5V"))
 (segment (start 45.276 108.666) (end 48.6 108.666) (width 0.6) (layer "F.Cu") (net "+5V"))
 (segment (start 48.6 108.666) (end 49.6 109.666) (width 0.6) (layer "F.Cu") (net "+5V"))
 (via (at 50.276 109.666) (size 0.6) (drill 0.3) (layers "F.Cu" "B.Cu") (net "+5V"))
 (segment (start 101.346 101.6) (end 101.346 33.274) (width 0.6) (layer "B.Cu") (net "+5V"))
 (segment (start 50.338 109.728) (end 93.218 109.728) (width 0.6) (layer "B.Cu") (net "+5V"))
 (segment (start 99.218 31.146) (end 90.896 31.146) (width 0.6) (layer "B.Cu") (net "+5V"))
 (segment (start 50.276 109.666) (end 50.338 109.728) (width 0.6) (layer "B.Cu") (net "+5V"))
 (segment (start 93.218 109.728) (end 101.346 101.6) (width 0.6) (layer "B.Cu") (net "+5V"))
 (segment (start 101.346 33.274) (end 99.218 31.146) (width 0.6) (layer "B.Cu") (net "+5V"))
 (segment (start 45.276 106.666) (end 50.575999 106.666) (width 0.4) (layer "F.Cu") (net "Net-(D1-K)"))
 (segment (start 45.276 77.966) (end 50.575999 77.966) (width 0.4) (layer "F.Cu") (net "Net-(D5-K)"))
 (segment (start 53.976 77.966) (end 56.92 77.966) (width 0.4) (layer "F.Cu") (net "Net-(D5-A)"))
 (segment (start 45.276 90.366) (end 50.575999 90.366) (width 0.4) (layer "F.Cu") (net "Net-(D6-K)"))
 (segment (start 69.276 93.366) (end 67.54 93.366) (width 0.4) (layer "F.Cu") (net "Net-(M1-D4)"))
 (segment (start 71.276 41.306) (end 70.276 42.306) (width 0.4) (layer "F.Cu") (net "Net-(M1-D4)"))
 (segment (start 70.276 92.366) (end 69.276 93.366) (width 0.4) (layer "F.Cu") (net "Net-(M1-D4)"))
 (segment (start 67.54 90.366) (end 67.54 93.366) (width 0.4) (layer "F.Cu") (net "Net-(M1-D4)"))
 (segment (start 48.6 92.366) (end 45.276 92.366) (width 0.4) (layer "F.Cu") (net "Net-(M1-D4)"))
 (segment (start 70.276 42.306) (end 70.276 92.366) (width 0.4) (layer "F.Cu") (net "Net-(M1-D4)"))
 (segment (start 67.54 93.366) (end 49.6 93.366) (width 0.4) (layer "F.Cu") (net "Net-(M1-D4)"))
 (segment (start 75.661 41.306) (end 71.276 41.306) (width 0.4) (layer "F.Cu") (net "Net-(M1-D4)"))
 (segment (start 49.6 93.366) (end 48.6 92.366) (width 0.4) (layer "F.Cu") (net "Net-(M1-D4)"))
 (segment (start 69.276 79.966) (end 68.276 80.966) (width 0.4) (layer "F.Cu") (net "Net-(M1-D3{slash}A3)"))
 (segment (start 75.661 38.766) (end 70.276 38.766) (width 0.4) (layer "F.Cu") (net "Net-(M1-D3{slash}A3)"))
 (segment (start 70.276 38.766) (end 69.276 39.766) (width 0.4) (layer "F.Cu") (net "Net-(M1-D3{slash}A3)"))
 (segment (start 67.54 80.966) (end 49.6 80.966) (width 0.4) (layer "F.Cu") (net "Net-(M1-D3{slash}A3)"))
 (segment (start 67.54 77.966) (end 67.54 80.966) (width 0.4) (layer "F.Cu") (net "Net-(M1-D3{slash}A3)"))
 (segment (start 68.276 80.966) (end 67.54 80.966) (width 0.4) (layer "F.Cu") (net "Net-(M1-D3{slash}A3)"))
 (segment (start 69.276 39.766) (end 69.276 79.966) (width 0.4) (layer "F.Cu") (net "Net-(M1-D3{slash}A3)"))
 (segment (start 48.6 79.966) (end 45.276 79.966) (width 0.4) (layer "F.Cu") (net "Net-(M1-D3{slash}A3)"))
 (segment (start 49.6 80.966) (end 48.6 79.966) (width 0.4) (layer "F.Cu") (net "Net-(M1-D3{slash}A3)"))
 (segment (start 45.276 65.566) (end 50.575999 65.566) (width 0.4) (layer "F.Cu") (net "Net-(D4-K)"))
 (segment (start 67.276 68.566) (end 49.6 68.566) (width 0.4) (layer "F.Cu") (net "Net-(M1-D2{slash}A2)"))
 (segment (start 68.276 37.226) (end 68.276 67.566) (width 0.4) (layer "F.Cu") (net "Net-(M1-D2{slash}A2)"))
 (segment (start 75.661 36.226) (end 69.276 36.226) (width 0.4) (layer "F.Cu") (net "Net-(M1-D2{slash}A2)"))
 (segment (start 48.6 67.566) (end 45.276 67.566) (width 0.4) (layer "F.Cu") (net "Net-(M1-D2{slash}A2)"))
 (segment (start 68.276 67.566) (end 67.276 68.566) (width 0.4) (layer "F.Cu") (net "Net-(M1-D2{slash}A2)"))
 (segment (start 69.276 36.226) (end 68.276 37.226) (width 0.4) (layer "F.Cu") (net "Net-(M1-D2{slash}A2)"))
 (segment (start 49.6 68.566) (end 48.6 67.566) (width 0.4) (layer "F.Cu") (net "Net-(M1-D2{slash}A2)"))
 (segment (start 53.976 106.666) (end 56.92 106.666) (width 0.4) (layer "F.Cu") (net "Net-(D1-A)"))
 (segment (start 53.976 51.166) (end 56.92 51.166) (width 0.4) (layer "F.Cu") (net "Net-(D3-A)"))
 (segment (start 53.976 65.566) (end 56.92 65.566) (width 0.4) (layer "F.Cu") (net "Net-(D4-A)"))
 (segment (start 45.276 36.766) (end 50.575999 36.766) (width 0.4) (layer "F.Cu") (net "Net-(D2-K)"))
 (segment (start 53.976 36.766) (end 56.92 36.766) (width 0.4) (layer "F.Cu") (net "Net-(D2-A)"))
 (segment (start 53.976 90.366) (end 56.92 90.366) (width 0.4) (layer "F.Cu") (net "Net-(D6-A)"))
 (segment (start 45.276 32.766) (end 48.6 32.766) (width 0.4) (layer "F.Cu") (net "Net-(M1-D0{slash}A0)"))
 (segment (start 50.22 31.146) (end 75.661 31.146) (width 0.4) (layer "F.Cu") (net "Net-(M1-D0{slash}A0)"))
 (segment (start 48.6 32.766) (end 50.22 31.146) (width 0.4) (layer "F.Cu") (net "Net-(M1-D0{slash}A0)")))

